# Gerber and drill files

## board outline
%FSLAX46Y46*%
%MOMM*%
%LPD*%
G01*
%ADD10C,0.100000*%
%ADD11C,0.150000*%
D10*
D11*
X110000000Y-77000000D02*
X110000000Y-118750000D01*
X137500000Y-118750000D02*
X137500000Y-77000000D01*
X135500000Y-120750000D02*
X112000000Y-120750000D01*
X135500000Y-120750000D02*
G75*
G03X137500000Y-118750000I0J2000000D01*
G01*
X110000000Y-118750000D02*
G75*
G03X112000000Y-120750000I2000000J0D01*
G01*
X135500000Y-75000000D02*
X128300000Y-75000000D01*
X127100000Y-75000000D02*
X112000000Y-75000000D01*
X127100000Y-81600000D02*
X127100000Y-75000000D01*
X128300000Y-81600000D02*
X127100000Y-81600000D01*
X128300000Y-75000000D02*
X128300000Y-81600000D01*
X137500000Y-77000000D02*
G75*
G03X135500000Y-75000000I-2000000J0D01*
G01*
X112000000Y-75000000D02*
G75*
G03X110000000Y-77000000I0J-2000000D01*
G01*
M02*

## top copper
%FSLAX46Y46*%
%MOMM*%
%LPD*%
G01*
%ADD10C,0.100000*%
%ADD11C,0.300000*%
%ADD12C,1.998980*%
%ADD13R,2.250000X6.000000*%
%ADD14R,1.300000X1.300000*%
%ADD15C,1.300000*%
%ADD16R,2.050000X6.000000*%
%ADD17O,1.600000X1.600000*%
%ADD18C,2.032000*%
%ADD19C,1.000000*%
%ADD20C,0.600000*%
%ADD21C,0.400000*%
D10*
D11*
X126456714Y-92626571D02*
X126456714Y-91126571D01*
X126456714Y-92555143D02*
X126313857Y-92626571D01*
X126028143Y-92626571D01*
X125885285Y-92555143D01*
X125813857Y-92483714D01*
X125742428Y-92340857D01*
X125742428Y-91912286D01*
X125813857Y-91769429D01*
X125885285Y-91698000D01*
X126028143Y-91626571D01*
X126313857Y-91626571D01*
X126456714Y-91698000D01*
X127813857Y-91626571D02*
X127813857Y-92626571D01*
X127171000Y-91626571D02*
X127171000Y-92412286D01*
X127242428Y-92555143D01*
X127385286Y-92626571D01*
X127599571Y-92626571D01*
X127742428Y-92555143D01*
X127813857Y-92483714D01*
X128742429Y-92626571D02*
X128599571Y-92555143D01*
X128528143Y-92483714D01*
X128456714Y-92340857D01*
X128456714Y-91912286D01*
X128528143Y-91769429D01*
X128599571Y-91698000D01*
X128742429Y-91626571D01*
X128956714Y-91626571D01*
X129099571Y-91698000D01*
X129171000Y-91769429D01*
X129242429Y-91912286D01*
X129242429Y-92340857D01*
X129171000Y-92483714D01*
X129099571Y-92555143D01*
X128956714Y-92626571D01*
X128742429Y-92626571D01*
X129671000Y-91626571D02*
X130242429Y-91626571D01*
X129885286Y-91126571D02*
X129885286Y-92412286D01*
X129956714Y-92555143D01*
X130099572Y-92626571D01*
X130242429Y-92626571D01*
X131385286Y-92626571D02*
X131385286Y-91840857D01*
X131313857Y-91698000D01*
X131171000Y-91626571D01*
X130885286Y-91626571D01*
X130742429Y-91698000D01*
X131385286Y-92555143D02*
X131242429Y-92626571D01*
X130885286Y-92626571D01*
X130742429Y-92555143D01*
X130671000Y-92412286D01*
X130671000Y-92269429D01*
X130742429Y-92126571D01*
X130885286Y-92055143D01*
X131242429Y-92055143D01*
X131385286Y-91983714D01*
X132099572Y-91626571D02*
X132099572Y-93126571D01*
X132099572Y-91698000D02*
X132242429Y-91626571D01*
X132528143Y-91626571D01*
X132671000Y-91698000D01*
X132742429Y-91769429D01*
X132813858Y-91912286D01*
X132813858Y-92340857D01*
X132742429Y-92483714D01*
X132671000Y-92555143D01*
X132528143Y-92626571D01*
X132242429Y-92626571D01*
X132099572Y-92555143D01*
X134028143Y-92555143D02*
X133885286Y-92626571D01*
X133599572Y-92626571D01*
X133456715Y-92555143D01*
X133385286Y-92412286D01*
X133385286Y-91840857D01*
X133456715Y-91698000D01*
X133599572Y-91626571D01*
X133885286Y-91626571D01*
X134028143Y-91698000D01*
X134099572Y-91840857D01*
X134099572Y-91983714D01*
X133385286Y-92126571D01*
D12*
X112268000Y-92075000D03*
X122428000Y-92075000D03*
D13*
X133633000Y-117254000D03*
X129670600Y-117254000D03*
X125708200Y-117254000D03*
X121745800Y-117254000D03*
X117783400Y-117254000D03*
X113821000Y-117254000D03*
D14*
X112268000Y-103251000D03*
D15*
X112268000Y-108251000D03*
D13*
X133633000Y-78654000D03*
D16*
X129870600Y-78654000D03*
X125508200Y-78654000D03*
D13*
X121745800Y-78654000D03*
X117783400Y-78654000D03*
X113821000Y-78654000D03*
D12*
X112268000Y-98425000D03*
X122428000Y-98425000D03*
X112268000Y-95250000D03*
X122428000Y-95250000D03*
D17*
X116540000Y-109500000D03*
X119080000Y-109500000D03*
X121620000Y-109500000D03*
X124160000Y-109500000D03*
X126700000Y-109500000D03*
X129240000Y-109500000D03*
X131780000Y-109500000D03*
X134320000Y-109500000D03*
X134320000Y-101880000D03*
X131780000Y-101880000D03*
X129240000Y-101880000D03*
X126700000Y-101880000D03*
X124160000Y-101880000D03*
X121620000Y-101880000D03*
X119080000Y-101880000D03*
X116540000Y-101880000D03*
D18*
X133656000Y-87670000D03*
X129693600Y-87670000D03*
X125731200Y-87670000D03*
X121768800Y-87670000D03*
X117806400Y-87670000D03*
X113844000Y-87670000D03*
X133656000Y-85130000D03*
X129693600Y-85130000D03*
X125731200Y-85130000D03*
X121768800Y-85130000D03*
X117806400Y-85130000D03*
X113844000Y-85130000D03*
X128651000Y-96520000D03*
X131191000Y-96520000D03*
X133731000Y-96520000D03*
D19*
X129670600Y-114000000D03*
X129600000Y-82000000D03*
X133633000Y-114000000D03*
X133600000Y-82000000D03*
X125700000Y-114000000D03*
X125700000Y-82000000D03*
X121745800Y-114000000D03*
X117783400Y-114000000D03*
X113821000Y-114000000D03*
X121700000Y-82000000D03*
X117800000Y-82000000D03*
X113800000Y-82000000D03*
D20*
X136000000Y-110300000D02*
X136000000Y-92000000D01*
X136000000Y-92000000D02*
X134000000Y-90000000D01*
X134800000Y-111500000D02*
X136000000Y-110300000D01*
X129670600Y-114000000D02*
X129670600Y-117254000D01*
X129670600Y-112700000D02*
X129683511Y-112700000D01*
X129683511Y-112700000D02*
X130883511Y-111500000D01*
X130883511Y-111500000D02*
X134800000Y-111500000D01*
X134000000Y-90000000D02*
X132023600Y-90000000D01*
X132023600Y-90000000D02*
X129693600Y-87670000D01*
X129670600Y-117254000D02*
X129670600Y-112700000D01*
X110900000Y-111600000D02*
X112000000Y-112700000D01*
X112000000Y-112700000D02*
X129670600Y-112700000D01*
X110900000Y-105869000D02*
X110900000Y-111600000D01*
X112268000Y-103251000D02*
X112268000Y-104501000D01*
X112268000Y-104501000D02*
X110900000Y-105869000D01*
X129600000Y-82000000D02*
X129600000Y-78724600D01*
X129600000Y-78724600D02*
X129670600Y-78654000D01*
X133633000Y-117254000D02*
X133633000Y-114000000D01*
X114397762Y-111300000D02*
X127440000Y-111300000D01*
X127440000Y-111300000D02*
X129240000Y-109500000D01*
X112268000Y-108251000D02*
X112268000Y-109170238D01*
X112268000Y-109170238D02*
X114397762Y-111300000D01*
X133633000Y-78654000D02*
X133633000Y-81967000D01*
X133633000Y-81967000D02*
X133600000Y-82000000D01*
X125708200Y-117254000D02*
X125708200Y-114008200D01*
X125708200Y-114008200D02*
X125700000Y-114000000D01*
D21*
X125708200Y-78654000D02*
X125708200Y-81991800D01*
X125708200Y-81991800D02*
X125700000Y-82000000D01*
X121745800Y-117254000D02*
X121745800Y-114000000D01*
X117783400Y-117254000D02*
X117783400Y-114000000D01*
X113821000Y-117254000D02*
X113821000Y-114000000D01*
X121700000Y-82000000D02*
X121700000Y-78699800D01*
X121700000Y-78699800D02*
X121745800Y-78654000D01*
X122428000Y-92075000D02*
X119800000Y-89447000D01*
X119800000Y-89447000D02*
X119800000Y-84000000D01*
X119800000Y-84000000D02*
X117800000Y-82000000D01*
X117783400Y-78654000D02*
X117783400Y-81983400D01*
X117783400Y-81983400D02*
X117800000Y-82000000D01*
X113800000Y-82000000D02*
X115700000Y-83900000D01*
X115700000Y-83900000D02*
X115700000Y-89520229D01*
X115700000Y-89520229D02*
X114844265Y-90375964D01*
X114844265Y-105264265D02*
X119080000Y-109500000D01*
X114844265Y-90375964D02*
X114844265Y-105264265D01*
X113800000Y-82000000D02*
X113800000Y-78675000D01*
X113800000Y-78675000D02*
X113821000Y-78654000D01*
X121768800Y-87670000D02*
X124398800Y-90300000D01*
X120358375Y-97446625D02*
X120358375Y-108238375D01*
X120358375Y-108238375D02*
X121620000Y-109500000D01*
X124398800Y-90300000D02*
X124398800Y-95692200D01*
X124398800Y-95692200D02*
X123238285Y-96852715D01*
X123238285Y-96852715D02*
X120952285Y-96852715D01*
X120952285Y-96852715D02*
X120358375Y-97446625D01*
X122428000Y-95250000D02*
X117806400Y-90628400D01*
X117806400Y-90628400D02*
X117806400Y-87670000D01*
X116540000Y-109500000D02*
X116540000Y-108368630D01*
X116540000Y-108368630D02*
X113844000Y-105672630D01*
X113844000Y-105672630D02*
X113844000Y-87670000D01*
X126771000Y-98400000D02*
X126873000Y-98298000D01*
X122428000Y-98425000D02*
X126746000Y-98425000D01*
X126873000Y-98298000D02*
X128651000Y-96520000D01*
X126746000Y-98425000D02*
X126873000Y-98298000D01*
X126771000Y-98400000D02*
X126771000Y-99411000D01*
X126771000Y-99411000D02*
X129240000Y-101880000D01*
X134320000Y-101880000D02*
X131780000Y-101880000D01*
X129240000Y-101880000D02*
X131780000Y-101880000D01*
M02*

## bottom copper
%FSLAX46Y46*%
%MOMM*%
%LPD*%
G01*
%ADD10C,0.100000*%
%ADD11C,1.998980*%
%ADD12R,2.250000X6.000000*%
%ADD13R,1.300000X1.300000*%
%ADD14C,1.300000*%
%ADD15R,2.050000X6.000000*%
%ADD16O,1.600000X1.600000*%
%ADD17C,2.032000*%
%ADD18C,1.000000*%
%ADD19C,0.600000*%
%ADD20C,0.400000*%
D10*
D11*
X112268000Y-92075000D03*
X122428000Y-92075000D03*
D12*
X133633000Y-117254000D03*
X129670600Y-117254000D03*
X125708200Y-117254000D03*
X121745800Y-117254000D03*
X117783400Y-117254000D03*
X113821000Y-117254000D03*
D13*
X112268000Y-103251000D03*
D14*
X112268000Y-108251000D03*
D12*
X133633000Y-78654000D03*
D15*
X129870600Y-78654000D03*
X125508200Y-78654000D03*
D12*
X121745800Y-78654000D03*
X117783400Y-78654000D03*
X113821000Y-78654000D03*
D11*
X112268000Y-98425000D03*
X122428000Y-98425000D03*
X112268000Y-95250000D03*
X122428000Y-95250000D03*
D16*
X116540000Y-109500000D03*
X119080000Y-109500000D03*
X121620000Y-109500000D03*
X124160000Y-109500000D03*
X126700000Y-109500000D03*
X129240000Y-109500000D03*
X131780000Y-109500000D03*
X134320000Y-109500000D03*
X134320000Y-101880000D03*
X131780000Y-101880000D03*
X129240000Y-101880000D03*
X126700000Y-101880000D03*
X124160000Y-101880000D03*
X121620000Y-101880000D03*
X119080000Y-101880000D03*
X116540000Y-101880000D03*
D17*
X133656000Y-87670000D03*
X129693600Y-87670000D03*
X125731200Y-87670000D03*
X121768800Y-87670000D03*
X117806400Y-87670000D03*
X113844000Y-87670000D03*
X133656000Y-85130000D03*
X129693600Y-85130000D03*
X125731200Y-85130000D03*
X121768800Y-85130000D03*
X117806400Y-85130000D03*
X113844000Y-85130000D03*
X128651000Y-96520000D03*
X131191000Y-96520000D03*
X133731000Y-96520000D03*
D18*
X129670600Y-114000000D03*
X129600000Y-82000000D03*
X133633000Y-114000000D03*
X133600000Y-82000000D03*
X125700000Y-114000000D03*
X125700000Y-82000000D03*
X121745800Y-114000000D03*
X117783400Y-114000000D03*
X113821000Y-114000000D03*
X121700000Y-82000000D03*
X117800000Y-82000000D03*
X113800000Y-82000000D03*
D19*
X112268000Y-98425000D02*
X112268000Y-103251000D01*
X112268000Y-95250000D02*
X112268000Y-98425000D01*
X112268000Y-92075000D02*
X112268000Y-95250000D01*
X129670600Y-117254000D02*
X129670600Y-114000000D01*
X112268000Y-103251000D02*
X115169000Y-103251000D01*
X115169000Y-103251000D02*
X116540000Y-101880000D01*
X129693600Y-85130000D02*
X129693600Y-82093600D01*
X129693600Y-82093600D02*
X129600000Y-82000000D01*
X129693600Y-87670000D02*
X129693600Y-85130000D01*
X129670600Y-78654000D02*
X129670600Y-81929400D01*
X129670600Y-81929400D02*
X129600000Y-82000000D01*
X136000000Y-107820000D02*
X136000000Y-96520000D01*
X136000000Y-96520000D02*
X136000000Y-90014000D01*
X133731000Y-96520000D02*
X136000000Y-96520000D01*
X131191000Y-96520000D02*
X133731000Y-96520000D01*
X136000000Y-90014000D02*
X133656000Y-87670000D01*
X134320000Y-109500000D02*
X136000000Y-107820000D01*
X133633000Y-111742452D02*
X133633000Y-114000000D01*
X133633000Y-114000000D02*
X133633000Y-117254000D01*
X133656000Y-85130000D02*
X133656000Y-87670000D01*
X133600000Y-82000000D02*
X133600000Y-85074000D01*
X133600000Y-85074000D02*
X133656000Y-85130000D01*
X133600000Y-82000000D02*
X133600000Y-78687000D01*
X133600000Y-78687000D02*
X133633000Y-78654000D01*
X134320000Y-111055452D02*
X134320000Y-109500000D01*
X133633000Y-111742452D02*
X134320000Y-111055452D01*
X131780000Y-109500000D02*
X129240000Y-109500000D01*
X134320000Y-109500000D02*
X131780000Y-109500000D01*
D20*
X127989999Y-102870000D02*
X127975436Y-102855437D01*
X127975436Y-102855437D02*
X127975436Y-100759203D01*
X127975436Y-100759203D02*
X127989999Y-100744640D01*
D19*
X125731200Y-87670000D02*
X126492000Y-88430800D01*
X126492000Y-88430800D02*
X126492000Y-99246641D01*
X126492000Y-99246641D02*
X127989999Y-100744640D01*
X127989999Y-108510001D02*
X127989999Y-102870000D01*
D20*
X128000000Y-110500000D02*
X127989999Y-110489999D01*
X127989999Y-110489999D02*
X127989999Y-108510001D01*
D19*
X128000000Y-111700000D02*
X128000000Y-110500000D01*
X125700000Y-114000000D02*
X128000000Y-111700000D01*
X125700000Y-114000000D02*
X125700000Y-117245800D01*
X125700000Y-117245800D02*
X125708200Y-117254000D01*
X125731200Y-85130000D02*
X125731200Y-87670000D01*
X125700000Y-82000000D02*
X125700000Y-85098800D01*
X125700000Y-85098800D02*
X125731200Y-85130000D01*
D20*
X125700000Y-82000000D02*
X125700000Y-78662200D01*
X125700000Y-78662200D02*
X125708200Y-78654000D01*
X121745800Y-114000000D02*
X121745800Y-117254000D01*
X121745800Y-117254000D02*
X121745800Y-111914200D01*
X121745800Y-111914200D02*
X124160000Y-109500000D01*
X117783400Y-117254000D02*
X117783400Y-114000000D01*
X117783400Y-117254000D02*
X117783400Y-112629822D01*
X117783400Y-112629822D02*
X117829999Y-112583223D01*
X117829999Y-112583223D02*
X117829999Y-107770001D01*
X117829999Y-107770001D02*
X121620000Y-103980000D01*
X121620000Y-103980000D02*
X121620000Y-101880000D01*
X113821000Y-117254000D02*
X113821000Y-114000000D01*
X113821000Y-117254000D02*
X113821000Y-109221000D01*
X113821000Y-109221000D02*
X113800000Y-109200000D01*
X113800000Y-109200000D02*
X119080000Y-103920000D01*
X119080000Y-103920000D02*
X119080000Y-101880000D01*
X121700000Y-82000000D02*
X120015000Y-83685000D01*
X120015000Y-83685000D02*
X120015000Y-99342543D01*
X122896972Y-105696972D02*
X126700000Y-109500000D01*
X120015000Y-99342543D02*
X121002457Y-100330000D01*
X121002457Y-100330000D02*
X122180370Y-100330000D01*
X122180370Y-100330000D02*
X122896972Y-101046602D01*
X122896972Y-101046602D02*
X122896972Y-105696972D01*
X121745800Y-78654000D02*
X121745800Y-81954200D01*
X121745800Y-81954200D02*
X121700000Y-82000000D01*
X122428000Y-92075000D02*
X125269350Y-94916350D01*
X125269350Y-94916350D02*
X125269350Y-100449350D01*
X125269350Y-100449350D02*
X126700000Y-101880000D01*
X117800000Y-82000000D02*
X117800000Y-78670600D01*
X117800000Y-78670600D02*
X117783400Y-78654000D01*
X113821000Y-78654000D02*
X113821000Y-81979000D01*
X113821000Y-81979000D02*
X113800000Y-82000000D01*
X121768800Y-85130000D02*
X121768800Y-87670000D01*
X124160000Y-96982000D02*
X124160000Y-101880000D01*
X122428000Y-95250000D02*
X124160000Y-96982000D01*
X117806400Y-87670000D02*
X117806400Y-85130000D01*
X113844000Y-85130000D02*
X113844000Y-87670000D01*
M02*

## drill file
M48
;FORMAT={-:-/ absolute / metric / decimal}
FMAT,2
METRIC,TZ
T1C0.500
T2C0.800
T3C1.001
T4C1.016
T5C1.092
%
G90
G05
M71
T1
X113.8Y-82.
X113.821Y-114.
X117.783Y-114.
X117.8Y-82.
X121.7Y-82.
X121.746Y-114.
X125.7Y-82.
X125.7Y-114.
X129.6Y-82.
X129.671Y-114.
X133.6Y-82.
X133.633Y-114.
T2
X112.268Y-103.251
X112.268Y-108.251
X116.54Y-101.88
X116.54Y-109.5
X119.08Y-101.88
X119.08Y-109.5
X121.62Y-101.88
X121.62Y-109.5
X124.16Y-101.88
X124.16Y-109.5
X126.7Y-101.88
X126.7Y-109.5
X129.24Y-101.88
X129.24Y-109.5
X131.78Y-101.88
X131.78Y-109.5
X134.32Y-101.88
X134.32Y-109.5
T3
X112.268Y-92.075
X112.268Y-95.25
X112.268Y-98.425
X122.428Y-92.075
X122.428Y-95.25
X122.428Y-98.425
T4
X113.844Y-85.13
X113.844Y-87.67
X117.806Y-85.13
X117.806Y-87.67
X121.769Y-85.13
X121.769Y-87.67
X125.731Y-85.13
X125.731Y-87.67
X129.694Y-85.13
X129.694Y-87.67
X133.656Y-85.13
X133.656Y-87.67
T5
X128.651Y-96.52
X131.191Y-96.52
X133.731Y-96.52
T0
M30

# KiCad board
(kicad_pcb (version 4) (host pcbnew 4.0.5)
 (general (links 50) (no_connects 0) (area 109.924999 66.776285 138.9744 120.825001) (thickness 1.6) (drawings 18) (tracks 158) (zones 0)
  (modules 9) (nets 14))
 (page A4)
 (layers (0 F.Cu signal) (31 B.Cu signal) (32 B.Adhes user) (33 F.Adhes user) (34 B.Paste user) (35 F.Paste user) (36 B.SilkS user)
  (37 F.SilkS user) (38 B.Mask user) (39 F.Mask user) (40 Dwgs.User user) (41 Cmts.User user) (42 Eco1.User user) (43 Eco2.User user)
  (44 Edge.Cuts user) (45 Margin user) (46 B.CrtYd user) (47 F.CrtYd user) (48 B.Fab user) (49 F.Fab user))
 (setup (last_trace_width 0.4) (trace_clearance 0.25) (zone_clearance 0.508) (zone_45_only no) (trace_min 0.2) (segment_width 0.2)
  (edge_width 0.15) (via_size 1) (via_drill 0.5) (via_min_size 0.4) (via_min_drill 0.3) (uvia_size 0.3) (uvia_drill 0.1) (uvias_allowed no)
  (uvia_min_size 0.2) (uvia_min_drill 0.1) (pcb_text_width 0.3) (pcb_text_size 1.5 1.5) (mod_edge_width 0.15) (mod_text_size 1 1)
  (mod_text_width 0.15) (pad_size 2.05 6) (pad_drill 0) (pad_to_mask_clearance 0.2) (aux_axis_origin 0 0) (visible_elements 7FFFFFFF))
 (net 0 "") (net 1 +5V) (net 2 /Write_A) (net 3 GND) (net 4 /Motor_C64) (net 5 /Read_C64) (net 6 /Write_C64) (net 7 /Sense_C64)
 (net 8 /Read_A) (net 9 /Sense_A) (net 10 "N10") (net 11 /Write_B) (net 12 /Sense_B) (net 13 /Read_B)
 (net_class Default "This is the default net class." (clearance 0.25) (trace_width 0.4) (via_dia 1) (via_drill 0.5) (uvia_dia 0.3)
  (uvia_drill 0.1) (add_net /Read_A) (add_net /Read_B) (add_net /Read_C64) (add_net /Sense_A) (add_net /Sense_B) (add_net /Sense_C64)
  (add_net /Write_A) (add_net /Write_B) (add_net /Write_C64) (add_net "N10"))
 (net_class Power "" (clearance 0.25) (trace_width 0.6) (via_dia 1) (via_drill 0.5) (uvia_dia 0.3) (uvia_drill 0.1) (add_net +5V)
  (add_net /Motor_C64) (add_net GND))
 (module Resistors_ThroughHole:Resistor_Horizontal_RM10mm (layer F.Cu) (at 112.268 92.075)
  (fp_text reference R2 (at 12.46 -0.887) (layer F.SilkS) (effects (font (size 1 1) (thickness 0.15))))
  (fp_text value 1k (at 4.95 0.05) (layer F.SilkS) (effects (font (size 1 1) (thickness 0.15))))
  (pad 1 thru_hole circle (at 0 0) (size 1.99898 1.99898) (drill 1.00076) (layers *.Cu *.SilkS *.Mask) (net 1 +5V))
  (pad 2 thru_hole circle (at 10.16 0) (size 1.99898 1.99898) (drill 1.00076) (layers *.Cu *.SilkS *.Mask) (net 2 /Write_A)))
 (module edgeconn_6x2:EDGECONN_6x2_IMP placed (layer F.Cu) (at 123.6 117 180)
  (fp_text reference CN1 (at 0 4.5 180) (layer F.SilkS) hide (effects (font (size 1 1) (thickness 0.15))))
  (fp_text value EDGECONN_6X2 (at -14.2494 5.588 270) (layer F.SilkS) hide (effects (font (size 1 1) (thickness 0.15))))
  (pad 1 smd rect (at -10.033 -0.254 180) (size 2.25 6) (layers F.Cu F.Paste F.Mask) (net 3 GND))
  (pad 2 smd rect (at -6.0706 -0.254 180) (size 2.25 6) (layers F.Cu F.Paste F.Mask) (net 1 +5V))
  (pad 3 smd rect (at -2.1082 -0.254 180) (size 2.25 6) (layers F.Cu F.Paste F.Mask) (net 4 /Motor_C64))
  (pad 4 smd rect (at 1.8542 -0.254 180) (size 2.25 6) (layers F.Cu F.Paste F.Mask) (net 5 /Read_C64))
  (pad 5 smd rect (at 5.8166 -0.254 180) (size 2.25 6) (layers F.Cu F.Paste F.Mask) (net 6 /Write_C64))
  (pad 6 smd rect (at 9.779 -0.254 180) (size 2.25 6) (layers F.Cu F.Paste F.Mask) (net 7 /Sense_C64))
  (pad A smd rect (at -10.033 -0.254 180) (size 2.25 6) (layers B.Cu B.Paste B.Mask) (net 3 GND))
  (pad B smd rect (at -6.0706 -0.254 180) (size 2.25 6) (layers B.Cu B.Paste B.Mask) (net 1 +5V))
  (pad C smd rect (at -2.1082 -0.254 180) (size 2.25 6) (layers B.Cu B.Paste B.Mask) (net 4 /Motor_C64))
  (pad D smd rect (at 1.8542 -0.254 180) (size 2.25 6) (layers B.Cu B.Paste B.Mask) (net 5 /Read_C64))
  (pad E smd rect (at 5.8166 -0.254 180) (size 2.25 6) (layers B.Cu B.Paste B.Mask) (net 6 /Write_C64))
  (pad F smd rect (at 9.779 -0.254 180) (size 2.25 6) (layers B.Cu B.Paste B.Mask) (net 7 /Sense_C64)))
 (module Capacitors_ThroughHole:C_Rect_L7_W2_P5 (layer F.Cu) (at 112.268 103.251 270)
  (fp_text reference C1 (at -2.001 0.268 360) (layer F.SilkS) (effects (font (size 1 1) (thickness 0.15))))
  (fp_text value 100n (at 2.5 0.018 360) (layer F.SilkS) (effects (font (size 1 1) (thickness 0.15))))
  (pad 1 thru_hole rect (at 0 0 270) (size 1.3 1.3) (drill 0.8) (layers *.Cu *.Mask F.SilkS) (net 1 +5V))
  (pad 2 thru_hole circle (at 5 0 270) (size 1.3 1.3) (drill 0.8) (layers *.Cu *.Mask F.SilkS) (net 3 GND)))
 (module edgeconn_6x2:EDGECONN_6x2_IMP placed (layer F.Cu) (at 123.6 78.4 180)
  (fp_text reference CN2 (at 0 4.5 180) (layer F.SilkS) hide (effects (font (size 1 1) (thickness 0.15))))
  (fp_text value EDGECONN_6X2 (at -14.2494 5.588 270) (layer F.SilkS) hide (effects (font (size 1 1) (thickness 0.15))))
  (pad 1 smd rect (at -10.033 -0.254 180) (size 2.25 6) (layers F.Cu F.Paste F.Mask) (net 3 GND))
  (pad 2 smd rect (at -6.0706 -0.254 180) (size 2.05 6) (drill (offset -0.2 0)) (layers F.Cu F.Paste F.Mask) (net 1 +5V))
  (pad 3 smd rect (at -2.1082 -0.254 180) (size 2.05 6) (drill (offset 0.2 0)) (layers F.Cu F.Paste F.Mask) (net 4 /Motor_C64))
  (pad 4 smd rect (at 1.8542 -0.254 180) (size 2.25 6) (layers F.Cu F.Paste F.Mask) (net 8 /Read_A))
  (pad 5 smd rect (at 5.8166 -0.254 180) (size 2.25 6) (layers F.Cu F.Paste F.Mask) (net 2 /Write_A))
  (pad 6 smd rect (at 9.779 -0.254 180) (size 2.25 6) (layers F.Cu F.Paste F.Mask) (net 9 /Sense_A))
  (pad A smd rect (at -10.033 -0.254 180) (size 2.25 6) (layers B.Cu B.Paste B.Mask) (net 3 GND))
  (pad B smd rect (at -6.0706 -0.254 180) (size 2.05 6) (drill (offset -0.2 0)) (layers B.Cu B.Paste B.Mask) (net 1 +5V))
  (pad C smd rect (at -2.1082 -0.254 180) (size 2.05 6) (drill (offset 0.2 0)) (layers B.Cu B.Paste B.Mask) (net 4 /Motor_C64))
  (pad D smd rect (at 1.8542 -0.254 180) (size 2.25 6) (layers B.Cu B.Paste B.Mask) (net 8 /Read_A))
  (pad E smd rect (at 5.8166 -0.254 180) (size 2.25 6) (layers B.Cu B.Paste B.Mask) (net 2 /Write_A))
  (pad F smd rect (at 9.779 -0.254 180) (size 2.25 6) (layers B.Cu B.Paste B.Mask) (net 9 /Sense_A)))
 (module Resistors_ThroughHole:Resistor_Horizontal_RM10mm (layer F.Cu) (at 112.268 98.425)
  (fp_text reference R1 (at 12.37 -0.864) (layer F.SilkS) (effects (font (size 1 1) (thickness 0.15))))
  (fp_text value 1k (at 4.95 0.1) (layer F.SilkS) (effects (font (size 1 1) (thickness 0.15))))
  (pad 1 thru_hole circle (at 0 0) (size 1.99898 1.99898) (drill 1.00076) (layers *.Cu *.SilkS *.Mask) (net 1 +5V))
  (pad 2 thru_hole circle (at 10.16 0) (size 1.99898 1.99898) (drill 1.00076) (layers *.Cu *.SilkS *.Mask) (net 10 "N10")))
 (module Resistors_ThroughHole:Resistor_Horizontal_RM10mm (layer F.Cu) (at 112.268 95.25)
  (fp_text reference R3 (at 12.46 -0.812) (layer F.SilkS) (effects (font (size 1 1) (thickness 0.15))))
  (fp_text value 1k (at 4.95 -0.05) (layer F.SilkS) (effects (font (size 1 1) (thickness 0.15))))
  (pad 1 thru_hole circle (at 0 0) (size 1.99898 1.99898) (drill 1.00076) (layers *.Cu *.SilkS *.Mask) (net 1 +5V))
  (pad 2 thru_hole circle (at 10.16 0) (size 1.99898 1.99898) (drill 1.00076) (layers *.Cu *.SilkS *.Mask) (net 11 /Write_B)))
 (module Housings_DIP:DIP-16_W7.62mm (layer F.Cu) (at 116.54 109.5 90)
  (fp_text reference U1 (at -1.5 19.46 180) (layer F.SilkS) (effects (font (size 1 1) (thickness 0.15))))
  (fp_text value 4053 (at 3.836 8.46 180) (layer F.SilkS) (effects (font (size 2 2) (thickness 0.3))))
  (pad 1 thru_hole oval (at 0 0 90) (size 1.6 1.6) (drill 0.8) (layers *.Cu *.Mask F.SilkS) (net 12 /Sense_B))
  (pad 2 thru_hole oval (at 0 2.54 90) (size 1.6 1.6) (drill 0.8) (layers *.Cu *.Mask F.SilkS) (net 9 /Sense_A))
  (pad 3 thru_hole oval (at 0 5.08 90) (size 1.6 1.6) (drill 0.8) (layers *.Cu *.Mask F.SilkS) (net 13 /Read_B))
  (pad 4 thru_hole oval (at 0 7.62 90) (size 1.6 1.6) (drill 0.8) (layers *.Cu *.Mask F.SilkS) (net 5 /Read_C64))
  (pad 5 thru_hole oval (at 0 10.16 90) (size 1.6 1.6) (drill 0.8) (layers *.Cu *.Mask F.SilkS) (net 8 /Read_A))
  (pad 6 thru_hole oval (at 0 12.7 90) (size 1.6 1.6) (drill 0.8) (layers *.Cu *.Mask F.SilkS) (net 3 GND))
  (pad 7 thru_hole oval (at 0 15.24 90) (size 1.6 1.6) (drill 0.8) (layers *.Cu *.Mask F.SilkS) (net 3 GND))
  (pad 8 thru_hole oval (at 0 17.78 90) (size 1.6 1.6) (drill 0.8) (layers *.Cu *.Mask F.SilkS) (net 3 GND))
  (pad 9 thru_hole oval (at 7.62 17.78 90) (size 1.6 1.6) (drill 0.8) (layers *.Cu *.Mask F.SilkS) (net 10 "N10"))
  (pad 10 thru_hole oval (at 7.62 15.24 90) (size 1.6 1.6) (drill 0.8) (layers *.Cu *.Mask F.SilkS) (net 10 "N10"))
  (pad 11 thru_hole oval (at 7.62 12.7 90) (size 1.6 1.6) (drill 0.8) (layers *.Cu *.Mask F.SilkS) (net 10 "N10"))
  (pad 12 thru_hole oval (at 7.62 10.16 90) (size 1.6 1.6) (drill 0.8) (layers *.Cu *.Mask F.SilkS) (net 2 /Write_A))
  (pad 13 thru_hole oval (at 7.62 7.62 90) (size 1.6 1.6) (drill 0.8) (layers *.Cu *.Mask F.SilkS) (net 11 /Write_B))
  (pad 14 thru_hole oval (at 7.62 5.08 90) (size 1.6 1.6) (drill 0.8) (layers *.Cu *.Mask F.SilkS) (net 6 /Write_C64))
  (pad 15 thru_hole oval (at 7.62 2.54 90) (size 1.6 1.6) (drill 0.8) (layers *.Cu *.Mask F.SilkS) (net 7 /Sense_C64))
  (pad 16 thru_hole oval (at 7.62 0 90) (size 1.6 1.6) (drill 0.8) (layers *.Cu *.Mask F.SilkS) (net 1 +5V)))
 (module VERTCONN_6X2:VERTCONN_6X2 (layer F.Cu) (at 123.75 86.4)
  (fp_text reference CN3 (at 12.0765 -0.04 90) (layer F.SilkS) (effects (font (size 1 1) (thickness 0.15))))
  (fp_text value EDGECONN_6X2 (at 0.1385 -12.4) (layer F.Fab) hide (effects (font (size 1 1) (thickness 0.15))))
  (pad 1 thru_hole circle (at 9.906 1.27) (size 2.032 2.032) (drill 1.016) (layers *.Cu *.Mask) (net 3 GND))
  (pad 2 thru_hole circle (at 5.9436 1.27) (size 2.032 2.032) (drill 1.016) (layers *.Cu *.Mask) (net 1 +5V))
  (pad 3 thru_hole circle (at 1.9812 1.27) (size 2.032 2.032) (drill 1.016) (layers *.Cu *.Mask) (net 4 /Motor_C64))
  (pad 4 thru_hole circle (at -1.9812 1.27) (size 2.032 2.032) (drill 1.016) (layers *.Cu *.Mask) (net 13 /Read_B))
  (pad 5 thru_hole circle (at -5.9436 1.27) (size 2.032 2.032) (drill 1.016) (layers *.Cu *.Mask) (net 11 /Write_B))
  (pad 6 thru_hole circle (at -9.906 1.27) (size 2.032 2.032) (drill 1.016) (layers *.Cu *.Mask) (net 12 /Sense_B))
  (pad A thru_hole circle (at 9.906 -1.27) (size 2.032 2.032) (drill 1.016) (layers *.Cu *.Mask) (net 3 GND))
  (pad B thru_hole circle (at 5.9436 -1.27) (size 2.032 2.032) (drill 1.016) (layers *.Cu *.Mask) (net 1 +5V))
  (pad C thru_hole circle (at 1.9812 -1.27) (size 2.032 2.032) (drill 1.016) (layers *.Cu *.Mask) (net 4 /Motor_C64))
  (pad D thru_hole circle (at -1.9812 -1.27) (size 2.032 2.032) (drill 1.016) (layers *.Cu *.Mask) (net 13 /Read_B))
  (pad E thru_hole circle (at -5.9436 -1.27) (size 2.032 2.032) (drill 1.016) (layers *.Cu *.Mask) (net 11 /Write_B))
  (pad F thru_hole circle (at -9.906 -1.27) (size 2.032 2.032) (drill 1.016) (layers *.Cu *.Mask) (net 12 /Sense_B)))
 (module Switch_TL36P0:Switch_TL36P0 (layer F.Cu) (at 131.191 96.52)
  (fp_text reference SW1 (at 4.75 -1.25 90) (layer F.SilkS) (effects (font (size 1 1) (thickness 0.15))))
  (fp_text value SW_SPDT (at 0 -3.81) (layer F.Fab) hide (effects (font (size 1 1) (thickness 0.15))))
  (pad 1 thru_hole circle (at -2.54 0) (size 2.032 2.032) (drill 1.0922) (layers *.Cu *.Mask) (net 10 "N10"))
  (pad 2 thru_hole circle (at 0 0) (size 2.032 2.032) (drill 1.0922) (layers *.Cu *.Mask) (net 3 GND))
  (pad 3 thru_hole circle (at 2.54 0) (size 2.032 2.032) (drill 1.0922) (layers *.Cu *.Mask) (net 3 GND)))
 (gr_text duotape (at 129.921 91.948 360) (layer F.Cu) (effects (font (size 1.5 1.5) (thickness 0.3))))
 (gr_line (start 110 77) (end 110 118.75) (layer Edge.Cuts) (width 0.15))
 (gr_line (start 137.5 118.75) (end 137.5 77) (layer Edge.Cuts) (width 0.15))
 (gr_line (start 135.5 120.75) (end 112 120.75) (layer Edge.Cuts) (width 0.15))
 (gr_arc (start 135.5 118.75) (end 137.5 118.75) (angle 90) (layer Edge.Cuts) (width 0.15))
 (gr_arc (start 112 118.75) (end 112 120.75) (angle 90) (layer Edge.Cuts) (width 0.15))
 (gr_line (start 135.5 75) (end 128.3 75) (layer Edge.Cuts) (width 0.15))
 (gr_line (start 127.1 75) (end 112 75) (layer Edge.Cuts) (width 0.15))
 (gr_line (start 127.1 81.6) (end 127.1 75) (layer Edge.Cuts) (width 0.15))
 (gr_line (start 128.3 81.6) (end 127.1 81.6) (layer Edge.Cuts) (width 0.15))
 (gr_line (start 128.3 75) (end 128.3 81.6) (layer Edge.Cuts) (width 0.15))
 (gr_arc (start 135.5 77) (end 135.5 75) (angle 90) (layer Edge.Cuts) (width 0.15))
 (gr_arc (start 112 77) (end 110 77) (angle 90) (layer Edge.Cuts) (width 0.15))
 (segment (start 112.268 98.425) (end 112.268 103.251) (width 0.6) (layer B.Cu) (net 1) (status 30))
 (segment (start 112.268 95.25) (end 112.268 98.425) (width 0.6) (layer B.Cu) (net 1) (status 30))
 (segment (start 112.268 92.075) (end 112.268 95.25) (width 0.6) (layer B.Cu) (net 1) (status 30))
 (segment (start 136 110.3) (end 136 92) (width 0.6) (layer F.Cu) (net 1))
 (segment (start 136 92) (end 134 90) (width 0.6) (layer F.Cu) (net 1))
 (segment (start 134.8 111.5) (end 136 110.3) (width 0.6) (layer F.Cu) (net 1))
 (segment (start 129.6706 114) (end 129.6706 117.254) (width 0.6) (layer F.Cu) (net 1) (status 20))
 (segment (start 129.6706 117.254) (end 129.6706 114) (width 0.6) (layer B.Cu) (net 1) (status 10))
 (segment (start 112.268 103.251) (end 115.169 103.251) (width 0.6) (layer B.Cu) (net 1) (status 10))
 (segment (start 115.169 103.251) (end 116.54 101.88) (width 0.6) (layer B.Cu) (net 1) (status 20))
 (segment (start 129.6706 112.7) (end 129.683511 112.7) (width 0.6) (layer F.Cu) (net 1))
 (segment (start 129.683511 112.7) (end 130.883511 111.5) (width 0.6) (layer F.Cu) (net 1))
 (segment (start 130.883511 111.5) (end 134.8 111.5) (width 0.6) (layer F.Cu) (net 1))
 (segment (start 134 90) (end 132.0236 90) (width 0.6) (layer F.Cu) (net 1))
 (segment (start 132.0236 90) (end 129.6936 87.67) (width 0.6) (layer F.Cu) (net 1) (status 20))
 (segment (start 129.6706 117.254) (end 129.6706 112.7) (width 0.6) (layer F.Cu) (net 1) (status 10))
 (segment (start 110.9 111.6) (end 112 112.7) (width 0.6) (layer F.Cu) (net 1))
 (segment (start 112 112.7) (end 129.6706 112.7) (width 0.6) (layer F.Cu) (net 1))
 (segment (start 110.9 105.869) (end 110.9 111.6) (width 0.6) (layer F.Cu) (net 1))
 (segment (start 112.268 103.251) (end 112.268 104.501) (width 0.6) (layer F.Cu) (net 1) (status 10))
 (segment (start 112.268 104.501) (end 110.9 105.869) (width 0.6) (layer F.Cu) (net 1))
 (via (at 129.6706 114) (size 1) (drill 0.5) (layers F.Cu B.Cu) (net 1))
 (segment (start 129.6936 85.13) (end 129.6936 82.0936) (width 0.6) (layer B.Cu) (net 1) (status 10))
 (segment (start 129.6936 82.0936) (end 129.6 82) (width 0.6) (layer B.Cu) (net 1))
 (segment (start 129.6936 87.67) (end 129.6936 85.13) (width 0.6) (layer B.Cu) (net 1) (status 30))
 (segment (start 129.6 82) (end 129.6 78.7246) (width 0.6) (layer F.Cu) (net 1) (status 20))
 (segment (start 129.6 78.7246) (end 129.6706 78.654) (width 0.6) (layer F.Cu) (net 1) (status 30))
 (segment (start 129.6706 78.654) (end 129.6706 81.9294) (width 0.6) (layer B.Cu) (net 1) (status 10))
 (segment (start 129.6706 81.9294) (end 129.6 82) (width 0.6) (layer B.Cu) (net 1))
 (via (at 129.6 82) (size 1) (drill 0.5) (layers F.Cu B.Cu) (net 1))
 (segment (start 136 107.82) (end 136 96.52) (width 0.6) (layer B.Cu) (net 3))
 (segment (start 136 96.52) (end 136 90.014) (width 0.6) (layer B.Cu) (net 3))
 (segment (start 133.731 96.52) (end 136 96.52) (width 0.6) (layer B.Cu) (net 3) (status 10))
 (segment (start 131.191 96.52) (end 133.731 96.52) (width 0.6) (layer B.Cu) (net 3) (status 30))
 (segment (start 136 90.014) (end 133.656 87.67) (width 0.6) (layer B.Cu) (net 3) (status 20))
 (segment (start 134.32 109.5) (end 136 107.82) (width 0.6) (layer B.Cu) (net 3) (status 10))
 (segment (start 133.633 111.742452) (end 133.633 114) (width 0.6) (layer B.Cu) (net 3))
 (segment (start 133.633 114) (end 133.633 117.254) (width 0.6) (layer B.Cu) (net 3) (status 20))
 (segment (start 133.633 117.254) (end 133.633 114) (width 0.6) (layer F.Cu) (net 3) (status 10))
 (via (at 133.633 114) (size 1) (drill 0.5) (layers F.Cu B.Cu) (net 3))
 (segment (start 114.397762 111.3) (end 127.44 111.3) (width 0.6) (layer F.Cu) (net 3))
 (segment (start 127.44 111.3) (end 129.24 109.5) (width 0.6) (layer F.Cu) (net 3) (status 20))
 (segment (start 112.268 108.251) (end 112.268 109.170238) (width 0.6) (layer F.Cu) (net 3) (status 10))
 (segment (start 112.268 109.170238) (end 114.397762 111.3) (width 0.6) (layer F.Cu) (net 3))
 (segment (start 133.656 85.13) (end 133.656 87.67) (width 0.6) (layer B.Cu) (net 3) (status 30))
 (segment (start 133.6 82) (end 133.6 85.074) (width 0.6) (layer B.Cu) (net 3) (status 20))
 (segment (start 133.6 85.074) (end 133.656 85.13) (width 0.6) (layer B.Cu) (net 3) (status 30))
 (segment (start 133.6 82) (end 133.6 78.687) (width 0.6) (layer B.Cu) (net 3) (status 20))
 (segment (start 133.6 78.687) (end 133.633 78.654) (width 0.6) (layer B.Cu) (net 3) (status 30))
 (segment (start 133.633 78.654) (end 133.633 81.967) (width 0.6) (layer F.Cu) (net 3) (status 10))
 (segment (start 133.633 81.967) (end 133.6 82) (width 0.6) (layer F.Cu) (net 3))
 (via (at 133.6 82) (size 1) (drill 0.5) (layers F.Cu B.Cu) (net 3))
 (segment (start 134.32 111.055452) (end 134.32 109.5) (width 0.6) (layer B.Cu) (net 3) (status 20))
 (segment (start 133.633 111.742452) (end 134.32 111.055452) (width 0.6) (layer B.Cu) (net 3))
 (segment (start 131.78 109.5) (end 129.24 109.5) (width 0.6) (layer B.Cu) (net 3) (status 30))
 (segment (start 134.32 109.5) (end 131.78 109.5) (width 0.6) (layer B.Cu) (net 3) (status 30))
 (segment (start 127.989999 102.87) (end 127.975436 102.855437) (width 0.4) (layer B.Cu) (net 4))
 (segment (start 127.975436 102.855437) (end 127.975436 100.759203) (width 0.4) (layer B.Cu) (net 4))
 (segment (start 127.975436 100.759203) (end 127.989999 100.74464) (width 0.4) (layer B.Cu) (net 4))
 (segment (start 125.7312 87.67) (end 126.492 88.4308) (width 0.6) (layer B.Cu) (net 4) (status 10))
 (segment (start 126.492 88.4308) (end 126.492 99.246641) (width 0.6) (layer B.Cu) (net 4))
 (segment (start 126.492 99.246641) (end 127.989999 100.74464) (width 0.6) (layer B.Cu) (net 4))
 (segment (start 127.989999 108.510001) (end 127.989999 102.87) (width 0.6) (layer B.Cu) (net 4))
 (segment (start 128 110.5) (end 127.989999 110.489999) (width 0.4) (layer B.Cu) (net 4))
 (segment (start 127.989999 110.489999) (end 127.989999 108.510001) (width 0.4) (layer B.Cu) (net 4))
 (segment (start 128 111.7) (end 128 110.5) (width 0.6) (layer B.Cu) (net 4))
 (segment (start 125.7 114) (end 128 111.7) (width 0.6) (layer B.Cu) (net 4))
 (segment (start 125.7 114) (end 125.7 117.2458) (width 0.6) (layer B.Cu) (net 4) (status 20))
 (segment (start 125.7 117.2458) (end 125.7082 117.254) (width 0.6) (layer B.Cu) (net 4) (status 30))
 (segment (start 125.7082 117.254) (end 125.7082 114.0082) (width 0.6) (layer F.Cu) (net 4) (status 10))
 (via (at 125.7 114) (size 1) (drill 0.5) (layers F.Cu B.Cu) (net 4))
 (segment (start 125.7082 114.0082) (end 125.7 114) (width 0.6) (layer F.Cu) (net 4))
 (segment (start 125.7312 85.13) (end 125.7312 87.67) (width 0.6) (layer B.Cu) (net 4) (status 30))
 (segment (start 125.7 82) (end 125.7 85.0988) (width 0.6) (layer B.Cu) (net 4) (status 20))
 (segment (start 125.7 85.0988) (end 125.7312 85.13) (width 0.6) (layer B.Cu) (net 4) (status 30))
 (segment (start 125.7 82) (end 125.7 78.6622) (width 0.4) (layer B.Cu) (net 4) (status 20))
 (segment (start 125.7 78.6622) (end 125.7082 78.654) (width 0.4) (layer B.Cu) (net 4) (status 30))
 (segment (start 125.7082 78.654) (end 125.7082 81.9918) (width 0.4) (layer F.Cu) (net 4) (status 10))
 (segment (start 125.7082 81.9918) (end 125.7 82) (width 0.4) (layer F.Cu) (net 4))
 (via (at 125.7 82) (size 1) (drill 0.5) (layers F.Cu B.Cu) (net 4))
 (segment (start 121.7458 114) (end 121.7458 117.254) (width 0.4) (layer B.Cu) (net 5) (status 20))
 (segment (start 121.7458 117.254) (end 121.7458 114) (width 0.4) (layer F.Cu) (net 5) (status 10))
 (via (at 121.7458 114) (size 1) (drill 0.5) (layers F.Cu B.Cu) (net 5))
 (segment (start 121.7458 117.254) (end 121.7458 111.9142) (width 0.4) (layer B.Cu) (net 5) (status 10))
 (segment (start 121.7458 111.9142) (end 124.16 109.5) (width 0.4) (layer B.Cu) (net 5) (status 20))
 (segment (start 117.7834 117.254) (end 117.7834 114) (width 0.4) (layer B.Cu) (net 6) (status 10))
 (segment (start 117.7834 117.254) (end 117.7834 114) (width 0.4) (layer F.Cu) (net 6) (status 10))
 (via (at 117.7834 114) (size 1) (drill 0.5) (layers F.Cu B.Cu) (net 6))
 (segment (start 117.7834 117.254) (end 117.7834 112.629822) (width 0.4) (layer B.Cu) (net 6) (status 10))
 (segment (start 117.7834 112.629822) (end 117.829999 112.583223) (width 0.4) (layer B.Cu) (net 6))
 (segment (start 117.829999 112.583223) (end 117.829999 107.770001) (width 0.4) (layer B.Cu) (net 6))
 (segment (start 117.829999 107.770001) (end 121.62 103.98) (width 0.4) (layer B.Cu) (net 6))
 (segment (start 121.62 103.98) (end 121.62 101.88) (width 0.4) (layer B.Cu) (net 6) (status 20))
 (segment (start 113.821 117.254) (end 113.821 114) (width 0.4) (layer B.Cu) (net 7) (status 10))
 (segment (start 113.821 117.254) (end 113.821 114) (width 0.4) (layer F.Cu) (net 7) (status 10))
 (via (at 113.821 114) (size 1) (drill 0.5) (layers F.Cu B.Cu) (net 7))
 (segment (start 113.821 117.254) (end 113.821 109.221) (width 0.4) (layer B.Cu) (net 7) (status 10))
 (segment (start 113.821 109.221) (end 113.8 109.2) (width 0.4) (layer B.Cu) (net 7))
 (segment (start 113.8 109.2) (end 119.08 103.92) (width 0.4) (layer B.Cu) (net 7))
 (segment (start 119.08 103.92) (end 119.08 101.88) (width 0.4) (layer B.Cu) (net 7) (status 20))
 (segment (start 121.7 82) (end 120.015 83.685) (width 0.4) (layer B.Cu) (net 8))
 (segment (start 120.015 83.685) (end 120.015 99.342543) (width 0.4) (layer B.Cu) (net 8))
 (segment (start 122.896972 105.696972) (end 126.7 109.5) (width 0.4) (layer B.Cu) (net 8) (status 20))
 (segment (start 120.015 99.342543) (end 121.002457 100.33) (width 0.4) (layer B.Cu) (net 8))
 (segment (start 121.002457 100.33) (end 122.18037 100.33) (width 0.4) (layer B.Cu) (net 8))
 (segment (start 122.18037 100.33) (end 122.896972 101.046602) (width 0.4) (layer B.Cu) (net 8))
 (segment (start 122.896972 101.046602) (end 122.896972 105.696972) (width 0.4) (layer B.Cu) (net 8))
 (segment (start 121.7 82) (end 121.7 78.6998) (width 0.4) (layer F.Cu) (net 8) (status 20))
 (segment (start 121.7 78.6998) (end 121.7458 78.654) (width 0.4) (layer F.Cu) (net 8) (status 30))
 (segment (start 121.7458 78.654) (end 121.7458 81.9542) (width 0.4) (layer B.Cu) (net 8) (status 10))
 (segment (start 121.7458 81.9542) (end 121.7 82) (width 0.4) (layer B.Cu) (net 8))
 (via (at 121.7 82) (size 1) (drill 0.5) (layers F.Cu B.Cu) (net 8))
 (segment (start 122.428 92.075) (end 125.26935 94.91635) (width 0.4) (layer B.Cu) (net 2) (status 10))
 (segment (start 125.26935 94.91635) (end 125.26935 100.44935) (width 0.4) (layer B.Cu) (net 2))
 (segment (start 125.26935 100.44935) (end 126.7 101.88) (width 0.4) (layer B.Cu) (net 2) (status 20))
 (segment (start 122.428 92.075) (end 119.8 89.447) (width 0.4) (layer F.Cu) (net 2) (status 10))
 (segment (start 119.8 89.447) (end 119.8 84) (width 0.4) (layer F.Cu) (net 2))
 (segment (start 119.8 84) (end 117.8 82) (width 0.4) (layer F.Cu) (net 2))
 (segment (start 117.8 82) (end 117.8 78.6706) (width 0.4) (layer B.Cu) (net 2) (status 20))
 (segment (start 117.8 78.6706) (end 117.7834 78.654) (width 0.4) (layer B.Cu) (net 2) (status 30))
 (segment (start 117.7834 78.654) (end 117.7834 81.9834) (width 0.4) (layer F.Cu) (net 2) (status 10))
 (segment (start 117.7834 81.9834) (end 117.8 82) (width 0.4) (layer F.Cu) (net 2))
 (via (at 117.8 82) (size 1) (drill 0.5) (layers F.Cu B.Cu) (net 2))
 (segment (start 113.8 82) (end 115.7 83.9) (width 0.4) (layer F.Cu) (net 9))
 (segment (start 115.7 83.9) (end 115.7 89.520229) (width 0.4) (layer F.Cu) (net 9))
 (segment (start 115.7 89.520229) (end 114.844265 90.375964) (width 0.4) (layer F.Cu) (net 9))
 (segment (start 114.844265 105.264265) (end 119.08 109.5) (width 0.4) (layer F.Cu) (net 9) (status 20))
 (segment (start 114.844265 90.375964) (end 114.844265 105.264265) (width 0.4) (layer F.Cu) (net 9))
 (segment (start 113.8 82) (end 113.8 78.675) (width 0.4) (layer F.Cu) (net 9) (status 20))
 (segment (start 113.8 78.675) (end 113.821 78.654) (width 0.4) (layer F.Cu) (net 9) (status 30))
 (segment (start 113.821 78.654) (end 113.821 81.979) (width 0.4) (layer B.Cu) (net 9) (status 10))
 (segment (start 113.821 81.979) (end 113.8 82) (width 0.4) (layer B.Cu) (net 9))
 (via (at 113.8 82) (size 1) (drill 0.5) (layers F.Cu B.Cu) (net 9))
 (segment (start 121.7688 87.67) (end 124.3988 90.3) (width 0.4) (layer F.Cu) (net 13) (status 10))
 (segment (start 120.358375 97.446625) (end 120.358375 108.238375) (width 0.4) (layer F.Cu) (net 13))
 (segment (start 120.358375 108.238375) (end 121.62 109.5) (width 0.4) (layer F.Cu) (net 13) (status 20))
 (segment (start 124.3988 90.3) (end 124.3988 95.6922) (width 0.4) (layer F.Cu) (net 13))
 (segment (start 124.3988 95.6922) (end 123.238285 96.852715) (width 0.4) (layer F.Cu) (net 13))
 (segment (start 123.238285 96.852715) (end 120.952285 96.852715) (width 0.4) (layer F.Cu) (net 13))
 (segment (start 120.952285 96.852715) (end 120.358375 97.446625) (width 0.4) (layer F.Cu) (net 13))
 (segment (start 121.7688 85.13) (end 121.7688 87.67) (width 0.4) (layer B.Cu) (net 13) (status 30))
 (segment (start 124.16 96.982) (end 124.16 101.88) (width 0.4) (layer B.Cu) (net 11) (status 20))
 (segment (start 122.428 95.25) (end 124.16 96.982) (width 0.4) (layer B.Cu) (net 11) (status 10))
 (segment (start 122.428 95.25) (end 117.8064 90.6284) (width 0.4) (layer F.Cu) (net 11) (status 10))
 (segment (start 117.8064 90.6284) (end 117.8064 87.67) (width 0.4) (layer F.Cu) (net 11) (status 20))
 (segment (start 117.8064 87.67) (end 117.8064 85.13) (width 0.4) (layer B.Cu) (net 11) (status 30))
 (segment (start 116.54 109.5) (end 116.54 108.36863) (width 0.4) (layer F.Cu) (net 12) (status 10))
 (segment (start 116.54 108.36863) (end 113.844 105.67263) (width 0.4) (layer F.Cu) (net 12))
 (segment (start 113.844 105.67263) (end 113.844 87.67) (width 0.4) (layer F.Cu) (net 12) (status 20))
 (segment (start 113.844 85.13) (end 113.844 87.67) (width 0.4) (layer B.Cu) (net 12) (status 30))
 (segment (start 126.771 98.4) (end 126.873 98.298) (width 0.4) (layer F.Cu) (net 10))
 (segment (start 122.428 98.425) (end 126.746 98.425) (width 0.4) (layer F.Cu) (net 10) (status 10))
 (segment (start 126.873 98.298) (end 128.651 96.52) (width 0.4) (layer F.Cu) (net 10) (status 20))
 (segment (start 126.746 98.425) (end 126.873 98.298) (width 0.4) (layer F.Cu) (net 10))
 (segment (start 126.771 98.4) (end 126.771 99.411) (width 0.4) (layer F.Cu) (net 10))
 (segment (start 126.771 99.411) (end 129.24 101.88) (width 0.4) (layer F.Cu) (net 10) (status 20))
 (segment (start 134.32 101.88) (end 131.78 101.88) (width 0.4) (layer F.Cu) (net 10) (status 30))
 (segment (start 129.24 101.88) (end 131.78 101.88) (width 0.4) (layer F.Cu) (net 10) (status 30)))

